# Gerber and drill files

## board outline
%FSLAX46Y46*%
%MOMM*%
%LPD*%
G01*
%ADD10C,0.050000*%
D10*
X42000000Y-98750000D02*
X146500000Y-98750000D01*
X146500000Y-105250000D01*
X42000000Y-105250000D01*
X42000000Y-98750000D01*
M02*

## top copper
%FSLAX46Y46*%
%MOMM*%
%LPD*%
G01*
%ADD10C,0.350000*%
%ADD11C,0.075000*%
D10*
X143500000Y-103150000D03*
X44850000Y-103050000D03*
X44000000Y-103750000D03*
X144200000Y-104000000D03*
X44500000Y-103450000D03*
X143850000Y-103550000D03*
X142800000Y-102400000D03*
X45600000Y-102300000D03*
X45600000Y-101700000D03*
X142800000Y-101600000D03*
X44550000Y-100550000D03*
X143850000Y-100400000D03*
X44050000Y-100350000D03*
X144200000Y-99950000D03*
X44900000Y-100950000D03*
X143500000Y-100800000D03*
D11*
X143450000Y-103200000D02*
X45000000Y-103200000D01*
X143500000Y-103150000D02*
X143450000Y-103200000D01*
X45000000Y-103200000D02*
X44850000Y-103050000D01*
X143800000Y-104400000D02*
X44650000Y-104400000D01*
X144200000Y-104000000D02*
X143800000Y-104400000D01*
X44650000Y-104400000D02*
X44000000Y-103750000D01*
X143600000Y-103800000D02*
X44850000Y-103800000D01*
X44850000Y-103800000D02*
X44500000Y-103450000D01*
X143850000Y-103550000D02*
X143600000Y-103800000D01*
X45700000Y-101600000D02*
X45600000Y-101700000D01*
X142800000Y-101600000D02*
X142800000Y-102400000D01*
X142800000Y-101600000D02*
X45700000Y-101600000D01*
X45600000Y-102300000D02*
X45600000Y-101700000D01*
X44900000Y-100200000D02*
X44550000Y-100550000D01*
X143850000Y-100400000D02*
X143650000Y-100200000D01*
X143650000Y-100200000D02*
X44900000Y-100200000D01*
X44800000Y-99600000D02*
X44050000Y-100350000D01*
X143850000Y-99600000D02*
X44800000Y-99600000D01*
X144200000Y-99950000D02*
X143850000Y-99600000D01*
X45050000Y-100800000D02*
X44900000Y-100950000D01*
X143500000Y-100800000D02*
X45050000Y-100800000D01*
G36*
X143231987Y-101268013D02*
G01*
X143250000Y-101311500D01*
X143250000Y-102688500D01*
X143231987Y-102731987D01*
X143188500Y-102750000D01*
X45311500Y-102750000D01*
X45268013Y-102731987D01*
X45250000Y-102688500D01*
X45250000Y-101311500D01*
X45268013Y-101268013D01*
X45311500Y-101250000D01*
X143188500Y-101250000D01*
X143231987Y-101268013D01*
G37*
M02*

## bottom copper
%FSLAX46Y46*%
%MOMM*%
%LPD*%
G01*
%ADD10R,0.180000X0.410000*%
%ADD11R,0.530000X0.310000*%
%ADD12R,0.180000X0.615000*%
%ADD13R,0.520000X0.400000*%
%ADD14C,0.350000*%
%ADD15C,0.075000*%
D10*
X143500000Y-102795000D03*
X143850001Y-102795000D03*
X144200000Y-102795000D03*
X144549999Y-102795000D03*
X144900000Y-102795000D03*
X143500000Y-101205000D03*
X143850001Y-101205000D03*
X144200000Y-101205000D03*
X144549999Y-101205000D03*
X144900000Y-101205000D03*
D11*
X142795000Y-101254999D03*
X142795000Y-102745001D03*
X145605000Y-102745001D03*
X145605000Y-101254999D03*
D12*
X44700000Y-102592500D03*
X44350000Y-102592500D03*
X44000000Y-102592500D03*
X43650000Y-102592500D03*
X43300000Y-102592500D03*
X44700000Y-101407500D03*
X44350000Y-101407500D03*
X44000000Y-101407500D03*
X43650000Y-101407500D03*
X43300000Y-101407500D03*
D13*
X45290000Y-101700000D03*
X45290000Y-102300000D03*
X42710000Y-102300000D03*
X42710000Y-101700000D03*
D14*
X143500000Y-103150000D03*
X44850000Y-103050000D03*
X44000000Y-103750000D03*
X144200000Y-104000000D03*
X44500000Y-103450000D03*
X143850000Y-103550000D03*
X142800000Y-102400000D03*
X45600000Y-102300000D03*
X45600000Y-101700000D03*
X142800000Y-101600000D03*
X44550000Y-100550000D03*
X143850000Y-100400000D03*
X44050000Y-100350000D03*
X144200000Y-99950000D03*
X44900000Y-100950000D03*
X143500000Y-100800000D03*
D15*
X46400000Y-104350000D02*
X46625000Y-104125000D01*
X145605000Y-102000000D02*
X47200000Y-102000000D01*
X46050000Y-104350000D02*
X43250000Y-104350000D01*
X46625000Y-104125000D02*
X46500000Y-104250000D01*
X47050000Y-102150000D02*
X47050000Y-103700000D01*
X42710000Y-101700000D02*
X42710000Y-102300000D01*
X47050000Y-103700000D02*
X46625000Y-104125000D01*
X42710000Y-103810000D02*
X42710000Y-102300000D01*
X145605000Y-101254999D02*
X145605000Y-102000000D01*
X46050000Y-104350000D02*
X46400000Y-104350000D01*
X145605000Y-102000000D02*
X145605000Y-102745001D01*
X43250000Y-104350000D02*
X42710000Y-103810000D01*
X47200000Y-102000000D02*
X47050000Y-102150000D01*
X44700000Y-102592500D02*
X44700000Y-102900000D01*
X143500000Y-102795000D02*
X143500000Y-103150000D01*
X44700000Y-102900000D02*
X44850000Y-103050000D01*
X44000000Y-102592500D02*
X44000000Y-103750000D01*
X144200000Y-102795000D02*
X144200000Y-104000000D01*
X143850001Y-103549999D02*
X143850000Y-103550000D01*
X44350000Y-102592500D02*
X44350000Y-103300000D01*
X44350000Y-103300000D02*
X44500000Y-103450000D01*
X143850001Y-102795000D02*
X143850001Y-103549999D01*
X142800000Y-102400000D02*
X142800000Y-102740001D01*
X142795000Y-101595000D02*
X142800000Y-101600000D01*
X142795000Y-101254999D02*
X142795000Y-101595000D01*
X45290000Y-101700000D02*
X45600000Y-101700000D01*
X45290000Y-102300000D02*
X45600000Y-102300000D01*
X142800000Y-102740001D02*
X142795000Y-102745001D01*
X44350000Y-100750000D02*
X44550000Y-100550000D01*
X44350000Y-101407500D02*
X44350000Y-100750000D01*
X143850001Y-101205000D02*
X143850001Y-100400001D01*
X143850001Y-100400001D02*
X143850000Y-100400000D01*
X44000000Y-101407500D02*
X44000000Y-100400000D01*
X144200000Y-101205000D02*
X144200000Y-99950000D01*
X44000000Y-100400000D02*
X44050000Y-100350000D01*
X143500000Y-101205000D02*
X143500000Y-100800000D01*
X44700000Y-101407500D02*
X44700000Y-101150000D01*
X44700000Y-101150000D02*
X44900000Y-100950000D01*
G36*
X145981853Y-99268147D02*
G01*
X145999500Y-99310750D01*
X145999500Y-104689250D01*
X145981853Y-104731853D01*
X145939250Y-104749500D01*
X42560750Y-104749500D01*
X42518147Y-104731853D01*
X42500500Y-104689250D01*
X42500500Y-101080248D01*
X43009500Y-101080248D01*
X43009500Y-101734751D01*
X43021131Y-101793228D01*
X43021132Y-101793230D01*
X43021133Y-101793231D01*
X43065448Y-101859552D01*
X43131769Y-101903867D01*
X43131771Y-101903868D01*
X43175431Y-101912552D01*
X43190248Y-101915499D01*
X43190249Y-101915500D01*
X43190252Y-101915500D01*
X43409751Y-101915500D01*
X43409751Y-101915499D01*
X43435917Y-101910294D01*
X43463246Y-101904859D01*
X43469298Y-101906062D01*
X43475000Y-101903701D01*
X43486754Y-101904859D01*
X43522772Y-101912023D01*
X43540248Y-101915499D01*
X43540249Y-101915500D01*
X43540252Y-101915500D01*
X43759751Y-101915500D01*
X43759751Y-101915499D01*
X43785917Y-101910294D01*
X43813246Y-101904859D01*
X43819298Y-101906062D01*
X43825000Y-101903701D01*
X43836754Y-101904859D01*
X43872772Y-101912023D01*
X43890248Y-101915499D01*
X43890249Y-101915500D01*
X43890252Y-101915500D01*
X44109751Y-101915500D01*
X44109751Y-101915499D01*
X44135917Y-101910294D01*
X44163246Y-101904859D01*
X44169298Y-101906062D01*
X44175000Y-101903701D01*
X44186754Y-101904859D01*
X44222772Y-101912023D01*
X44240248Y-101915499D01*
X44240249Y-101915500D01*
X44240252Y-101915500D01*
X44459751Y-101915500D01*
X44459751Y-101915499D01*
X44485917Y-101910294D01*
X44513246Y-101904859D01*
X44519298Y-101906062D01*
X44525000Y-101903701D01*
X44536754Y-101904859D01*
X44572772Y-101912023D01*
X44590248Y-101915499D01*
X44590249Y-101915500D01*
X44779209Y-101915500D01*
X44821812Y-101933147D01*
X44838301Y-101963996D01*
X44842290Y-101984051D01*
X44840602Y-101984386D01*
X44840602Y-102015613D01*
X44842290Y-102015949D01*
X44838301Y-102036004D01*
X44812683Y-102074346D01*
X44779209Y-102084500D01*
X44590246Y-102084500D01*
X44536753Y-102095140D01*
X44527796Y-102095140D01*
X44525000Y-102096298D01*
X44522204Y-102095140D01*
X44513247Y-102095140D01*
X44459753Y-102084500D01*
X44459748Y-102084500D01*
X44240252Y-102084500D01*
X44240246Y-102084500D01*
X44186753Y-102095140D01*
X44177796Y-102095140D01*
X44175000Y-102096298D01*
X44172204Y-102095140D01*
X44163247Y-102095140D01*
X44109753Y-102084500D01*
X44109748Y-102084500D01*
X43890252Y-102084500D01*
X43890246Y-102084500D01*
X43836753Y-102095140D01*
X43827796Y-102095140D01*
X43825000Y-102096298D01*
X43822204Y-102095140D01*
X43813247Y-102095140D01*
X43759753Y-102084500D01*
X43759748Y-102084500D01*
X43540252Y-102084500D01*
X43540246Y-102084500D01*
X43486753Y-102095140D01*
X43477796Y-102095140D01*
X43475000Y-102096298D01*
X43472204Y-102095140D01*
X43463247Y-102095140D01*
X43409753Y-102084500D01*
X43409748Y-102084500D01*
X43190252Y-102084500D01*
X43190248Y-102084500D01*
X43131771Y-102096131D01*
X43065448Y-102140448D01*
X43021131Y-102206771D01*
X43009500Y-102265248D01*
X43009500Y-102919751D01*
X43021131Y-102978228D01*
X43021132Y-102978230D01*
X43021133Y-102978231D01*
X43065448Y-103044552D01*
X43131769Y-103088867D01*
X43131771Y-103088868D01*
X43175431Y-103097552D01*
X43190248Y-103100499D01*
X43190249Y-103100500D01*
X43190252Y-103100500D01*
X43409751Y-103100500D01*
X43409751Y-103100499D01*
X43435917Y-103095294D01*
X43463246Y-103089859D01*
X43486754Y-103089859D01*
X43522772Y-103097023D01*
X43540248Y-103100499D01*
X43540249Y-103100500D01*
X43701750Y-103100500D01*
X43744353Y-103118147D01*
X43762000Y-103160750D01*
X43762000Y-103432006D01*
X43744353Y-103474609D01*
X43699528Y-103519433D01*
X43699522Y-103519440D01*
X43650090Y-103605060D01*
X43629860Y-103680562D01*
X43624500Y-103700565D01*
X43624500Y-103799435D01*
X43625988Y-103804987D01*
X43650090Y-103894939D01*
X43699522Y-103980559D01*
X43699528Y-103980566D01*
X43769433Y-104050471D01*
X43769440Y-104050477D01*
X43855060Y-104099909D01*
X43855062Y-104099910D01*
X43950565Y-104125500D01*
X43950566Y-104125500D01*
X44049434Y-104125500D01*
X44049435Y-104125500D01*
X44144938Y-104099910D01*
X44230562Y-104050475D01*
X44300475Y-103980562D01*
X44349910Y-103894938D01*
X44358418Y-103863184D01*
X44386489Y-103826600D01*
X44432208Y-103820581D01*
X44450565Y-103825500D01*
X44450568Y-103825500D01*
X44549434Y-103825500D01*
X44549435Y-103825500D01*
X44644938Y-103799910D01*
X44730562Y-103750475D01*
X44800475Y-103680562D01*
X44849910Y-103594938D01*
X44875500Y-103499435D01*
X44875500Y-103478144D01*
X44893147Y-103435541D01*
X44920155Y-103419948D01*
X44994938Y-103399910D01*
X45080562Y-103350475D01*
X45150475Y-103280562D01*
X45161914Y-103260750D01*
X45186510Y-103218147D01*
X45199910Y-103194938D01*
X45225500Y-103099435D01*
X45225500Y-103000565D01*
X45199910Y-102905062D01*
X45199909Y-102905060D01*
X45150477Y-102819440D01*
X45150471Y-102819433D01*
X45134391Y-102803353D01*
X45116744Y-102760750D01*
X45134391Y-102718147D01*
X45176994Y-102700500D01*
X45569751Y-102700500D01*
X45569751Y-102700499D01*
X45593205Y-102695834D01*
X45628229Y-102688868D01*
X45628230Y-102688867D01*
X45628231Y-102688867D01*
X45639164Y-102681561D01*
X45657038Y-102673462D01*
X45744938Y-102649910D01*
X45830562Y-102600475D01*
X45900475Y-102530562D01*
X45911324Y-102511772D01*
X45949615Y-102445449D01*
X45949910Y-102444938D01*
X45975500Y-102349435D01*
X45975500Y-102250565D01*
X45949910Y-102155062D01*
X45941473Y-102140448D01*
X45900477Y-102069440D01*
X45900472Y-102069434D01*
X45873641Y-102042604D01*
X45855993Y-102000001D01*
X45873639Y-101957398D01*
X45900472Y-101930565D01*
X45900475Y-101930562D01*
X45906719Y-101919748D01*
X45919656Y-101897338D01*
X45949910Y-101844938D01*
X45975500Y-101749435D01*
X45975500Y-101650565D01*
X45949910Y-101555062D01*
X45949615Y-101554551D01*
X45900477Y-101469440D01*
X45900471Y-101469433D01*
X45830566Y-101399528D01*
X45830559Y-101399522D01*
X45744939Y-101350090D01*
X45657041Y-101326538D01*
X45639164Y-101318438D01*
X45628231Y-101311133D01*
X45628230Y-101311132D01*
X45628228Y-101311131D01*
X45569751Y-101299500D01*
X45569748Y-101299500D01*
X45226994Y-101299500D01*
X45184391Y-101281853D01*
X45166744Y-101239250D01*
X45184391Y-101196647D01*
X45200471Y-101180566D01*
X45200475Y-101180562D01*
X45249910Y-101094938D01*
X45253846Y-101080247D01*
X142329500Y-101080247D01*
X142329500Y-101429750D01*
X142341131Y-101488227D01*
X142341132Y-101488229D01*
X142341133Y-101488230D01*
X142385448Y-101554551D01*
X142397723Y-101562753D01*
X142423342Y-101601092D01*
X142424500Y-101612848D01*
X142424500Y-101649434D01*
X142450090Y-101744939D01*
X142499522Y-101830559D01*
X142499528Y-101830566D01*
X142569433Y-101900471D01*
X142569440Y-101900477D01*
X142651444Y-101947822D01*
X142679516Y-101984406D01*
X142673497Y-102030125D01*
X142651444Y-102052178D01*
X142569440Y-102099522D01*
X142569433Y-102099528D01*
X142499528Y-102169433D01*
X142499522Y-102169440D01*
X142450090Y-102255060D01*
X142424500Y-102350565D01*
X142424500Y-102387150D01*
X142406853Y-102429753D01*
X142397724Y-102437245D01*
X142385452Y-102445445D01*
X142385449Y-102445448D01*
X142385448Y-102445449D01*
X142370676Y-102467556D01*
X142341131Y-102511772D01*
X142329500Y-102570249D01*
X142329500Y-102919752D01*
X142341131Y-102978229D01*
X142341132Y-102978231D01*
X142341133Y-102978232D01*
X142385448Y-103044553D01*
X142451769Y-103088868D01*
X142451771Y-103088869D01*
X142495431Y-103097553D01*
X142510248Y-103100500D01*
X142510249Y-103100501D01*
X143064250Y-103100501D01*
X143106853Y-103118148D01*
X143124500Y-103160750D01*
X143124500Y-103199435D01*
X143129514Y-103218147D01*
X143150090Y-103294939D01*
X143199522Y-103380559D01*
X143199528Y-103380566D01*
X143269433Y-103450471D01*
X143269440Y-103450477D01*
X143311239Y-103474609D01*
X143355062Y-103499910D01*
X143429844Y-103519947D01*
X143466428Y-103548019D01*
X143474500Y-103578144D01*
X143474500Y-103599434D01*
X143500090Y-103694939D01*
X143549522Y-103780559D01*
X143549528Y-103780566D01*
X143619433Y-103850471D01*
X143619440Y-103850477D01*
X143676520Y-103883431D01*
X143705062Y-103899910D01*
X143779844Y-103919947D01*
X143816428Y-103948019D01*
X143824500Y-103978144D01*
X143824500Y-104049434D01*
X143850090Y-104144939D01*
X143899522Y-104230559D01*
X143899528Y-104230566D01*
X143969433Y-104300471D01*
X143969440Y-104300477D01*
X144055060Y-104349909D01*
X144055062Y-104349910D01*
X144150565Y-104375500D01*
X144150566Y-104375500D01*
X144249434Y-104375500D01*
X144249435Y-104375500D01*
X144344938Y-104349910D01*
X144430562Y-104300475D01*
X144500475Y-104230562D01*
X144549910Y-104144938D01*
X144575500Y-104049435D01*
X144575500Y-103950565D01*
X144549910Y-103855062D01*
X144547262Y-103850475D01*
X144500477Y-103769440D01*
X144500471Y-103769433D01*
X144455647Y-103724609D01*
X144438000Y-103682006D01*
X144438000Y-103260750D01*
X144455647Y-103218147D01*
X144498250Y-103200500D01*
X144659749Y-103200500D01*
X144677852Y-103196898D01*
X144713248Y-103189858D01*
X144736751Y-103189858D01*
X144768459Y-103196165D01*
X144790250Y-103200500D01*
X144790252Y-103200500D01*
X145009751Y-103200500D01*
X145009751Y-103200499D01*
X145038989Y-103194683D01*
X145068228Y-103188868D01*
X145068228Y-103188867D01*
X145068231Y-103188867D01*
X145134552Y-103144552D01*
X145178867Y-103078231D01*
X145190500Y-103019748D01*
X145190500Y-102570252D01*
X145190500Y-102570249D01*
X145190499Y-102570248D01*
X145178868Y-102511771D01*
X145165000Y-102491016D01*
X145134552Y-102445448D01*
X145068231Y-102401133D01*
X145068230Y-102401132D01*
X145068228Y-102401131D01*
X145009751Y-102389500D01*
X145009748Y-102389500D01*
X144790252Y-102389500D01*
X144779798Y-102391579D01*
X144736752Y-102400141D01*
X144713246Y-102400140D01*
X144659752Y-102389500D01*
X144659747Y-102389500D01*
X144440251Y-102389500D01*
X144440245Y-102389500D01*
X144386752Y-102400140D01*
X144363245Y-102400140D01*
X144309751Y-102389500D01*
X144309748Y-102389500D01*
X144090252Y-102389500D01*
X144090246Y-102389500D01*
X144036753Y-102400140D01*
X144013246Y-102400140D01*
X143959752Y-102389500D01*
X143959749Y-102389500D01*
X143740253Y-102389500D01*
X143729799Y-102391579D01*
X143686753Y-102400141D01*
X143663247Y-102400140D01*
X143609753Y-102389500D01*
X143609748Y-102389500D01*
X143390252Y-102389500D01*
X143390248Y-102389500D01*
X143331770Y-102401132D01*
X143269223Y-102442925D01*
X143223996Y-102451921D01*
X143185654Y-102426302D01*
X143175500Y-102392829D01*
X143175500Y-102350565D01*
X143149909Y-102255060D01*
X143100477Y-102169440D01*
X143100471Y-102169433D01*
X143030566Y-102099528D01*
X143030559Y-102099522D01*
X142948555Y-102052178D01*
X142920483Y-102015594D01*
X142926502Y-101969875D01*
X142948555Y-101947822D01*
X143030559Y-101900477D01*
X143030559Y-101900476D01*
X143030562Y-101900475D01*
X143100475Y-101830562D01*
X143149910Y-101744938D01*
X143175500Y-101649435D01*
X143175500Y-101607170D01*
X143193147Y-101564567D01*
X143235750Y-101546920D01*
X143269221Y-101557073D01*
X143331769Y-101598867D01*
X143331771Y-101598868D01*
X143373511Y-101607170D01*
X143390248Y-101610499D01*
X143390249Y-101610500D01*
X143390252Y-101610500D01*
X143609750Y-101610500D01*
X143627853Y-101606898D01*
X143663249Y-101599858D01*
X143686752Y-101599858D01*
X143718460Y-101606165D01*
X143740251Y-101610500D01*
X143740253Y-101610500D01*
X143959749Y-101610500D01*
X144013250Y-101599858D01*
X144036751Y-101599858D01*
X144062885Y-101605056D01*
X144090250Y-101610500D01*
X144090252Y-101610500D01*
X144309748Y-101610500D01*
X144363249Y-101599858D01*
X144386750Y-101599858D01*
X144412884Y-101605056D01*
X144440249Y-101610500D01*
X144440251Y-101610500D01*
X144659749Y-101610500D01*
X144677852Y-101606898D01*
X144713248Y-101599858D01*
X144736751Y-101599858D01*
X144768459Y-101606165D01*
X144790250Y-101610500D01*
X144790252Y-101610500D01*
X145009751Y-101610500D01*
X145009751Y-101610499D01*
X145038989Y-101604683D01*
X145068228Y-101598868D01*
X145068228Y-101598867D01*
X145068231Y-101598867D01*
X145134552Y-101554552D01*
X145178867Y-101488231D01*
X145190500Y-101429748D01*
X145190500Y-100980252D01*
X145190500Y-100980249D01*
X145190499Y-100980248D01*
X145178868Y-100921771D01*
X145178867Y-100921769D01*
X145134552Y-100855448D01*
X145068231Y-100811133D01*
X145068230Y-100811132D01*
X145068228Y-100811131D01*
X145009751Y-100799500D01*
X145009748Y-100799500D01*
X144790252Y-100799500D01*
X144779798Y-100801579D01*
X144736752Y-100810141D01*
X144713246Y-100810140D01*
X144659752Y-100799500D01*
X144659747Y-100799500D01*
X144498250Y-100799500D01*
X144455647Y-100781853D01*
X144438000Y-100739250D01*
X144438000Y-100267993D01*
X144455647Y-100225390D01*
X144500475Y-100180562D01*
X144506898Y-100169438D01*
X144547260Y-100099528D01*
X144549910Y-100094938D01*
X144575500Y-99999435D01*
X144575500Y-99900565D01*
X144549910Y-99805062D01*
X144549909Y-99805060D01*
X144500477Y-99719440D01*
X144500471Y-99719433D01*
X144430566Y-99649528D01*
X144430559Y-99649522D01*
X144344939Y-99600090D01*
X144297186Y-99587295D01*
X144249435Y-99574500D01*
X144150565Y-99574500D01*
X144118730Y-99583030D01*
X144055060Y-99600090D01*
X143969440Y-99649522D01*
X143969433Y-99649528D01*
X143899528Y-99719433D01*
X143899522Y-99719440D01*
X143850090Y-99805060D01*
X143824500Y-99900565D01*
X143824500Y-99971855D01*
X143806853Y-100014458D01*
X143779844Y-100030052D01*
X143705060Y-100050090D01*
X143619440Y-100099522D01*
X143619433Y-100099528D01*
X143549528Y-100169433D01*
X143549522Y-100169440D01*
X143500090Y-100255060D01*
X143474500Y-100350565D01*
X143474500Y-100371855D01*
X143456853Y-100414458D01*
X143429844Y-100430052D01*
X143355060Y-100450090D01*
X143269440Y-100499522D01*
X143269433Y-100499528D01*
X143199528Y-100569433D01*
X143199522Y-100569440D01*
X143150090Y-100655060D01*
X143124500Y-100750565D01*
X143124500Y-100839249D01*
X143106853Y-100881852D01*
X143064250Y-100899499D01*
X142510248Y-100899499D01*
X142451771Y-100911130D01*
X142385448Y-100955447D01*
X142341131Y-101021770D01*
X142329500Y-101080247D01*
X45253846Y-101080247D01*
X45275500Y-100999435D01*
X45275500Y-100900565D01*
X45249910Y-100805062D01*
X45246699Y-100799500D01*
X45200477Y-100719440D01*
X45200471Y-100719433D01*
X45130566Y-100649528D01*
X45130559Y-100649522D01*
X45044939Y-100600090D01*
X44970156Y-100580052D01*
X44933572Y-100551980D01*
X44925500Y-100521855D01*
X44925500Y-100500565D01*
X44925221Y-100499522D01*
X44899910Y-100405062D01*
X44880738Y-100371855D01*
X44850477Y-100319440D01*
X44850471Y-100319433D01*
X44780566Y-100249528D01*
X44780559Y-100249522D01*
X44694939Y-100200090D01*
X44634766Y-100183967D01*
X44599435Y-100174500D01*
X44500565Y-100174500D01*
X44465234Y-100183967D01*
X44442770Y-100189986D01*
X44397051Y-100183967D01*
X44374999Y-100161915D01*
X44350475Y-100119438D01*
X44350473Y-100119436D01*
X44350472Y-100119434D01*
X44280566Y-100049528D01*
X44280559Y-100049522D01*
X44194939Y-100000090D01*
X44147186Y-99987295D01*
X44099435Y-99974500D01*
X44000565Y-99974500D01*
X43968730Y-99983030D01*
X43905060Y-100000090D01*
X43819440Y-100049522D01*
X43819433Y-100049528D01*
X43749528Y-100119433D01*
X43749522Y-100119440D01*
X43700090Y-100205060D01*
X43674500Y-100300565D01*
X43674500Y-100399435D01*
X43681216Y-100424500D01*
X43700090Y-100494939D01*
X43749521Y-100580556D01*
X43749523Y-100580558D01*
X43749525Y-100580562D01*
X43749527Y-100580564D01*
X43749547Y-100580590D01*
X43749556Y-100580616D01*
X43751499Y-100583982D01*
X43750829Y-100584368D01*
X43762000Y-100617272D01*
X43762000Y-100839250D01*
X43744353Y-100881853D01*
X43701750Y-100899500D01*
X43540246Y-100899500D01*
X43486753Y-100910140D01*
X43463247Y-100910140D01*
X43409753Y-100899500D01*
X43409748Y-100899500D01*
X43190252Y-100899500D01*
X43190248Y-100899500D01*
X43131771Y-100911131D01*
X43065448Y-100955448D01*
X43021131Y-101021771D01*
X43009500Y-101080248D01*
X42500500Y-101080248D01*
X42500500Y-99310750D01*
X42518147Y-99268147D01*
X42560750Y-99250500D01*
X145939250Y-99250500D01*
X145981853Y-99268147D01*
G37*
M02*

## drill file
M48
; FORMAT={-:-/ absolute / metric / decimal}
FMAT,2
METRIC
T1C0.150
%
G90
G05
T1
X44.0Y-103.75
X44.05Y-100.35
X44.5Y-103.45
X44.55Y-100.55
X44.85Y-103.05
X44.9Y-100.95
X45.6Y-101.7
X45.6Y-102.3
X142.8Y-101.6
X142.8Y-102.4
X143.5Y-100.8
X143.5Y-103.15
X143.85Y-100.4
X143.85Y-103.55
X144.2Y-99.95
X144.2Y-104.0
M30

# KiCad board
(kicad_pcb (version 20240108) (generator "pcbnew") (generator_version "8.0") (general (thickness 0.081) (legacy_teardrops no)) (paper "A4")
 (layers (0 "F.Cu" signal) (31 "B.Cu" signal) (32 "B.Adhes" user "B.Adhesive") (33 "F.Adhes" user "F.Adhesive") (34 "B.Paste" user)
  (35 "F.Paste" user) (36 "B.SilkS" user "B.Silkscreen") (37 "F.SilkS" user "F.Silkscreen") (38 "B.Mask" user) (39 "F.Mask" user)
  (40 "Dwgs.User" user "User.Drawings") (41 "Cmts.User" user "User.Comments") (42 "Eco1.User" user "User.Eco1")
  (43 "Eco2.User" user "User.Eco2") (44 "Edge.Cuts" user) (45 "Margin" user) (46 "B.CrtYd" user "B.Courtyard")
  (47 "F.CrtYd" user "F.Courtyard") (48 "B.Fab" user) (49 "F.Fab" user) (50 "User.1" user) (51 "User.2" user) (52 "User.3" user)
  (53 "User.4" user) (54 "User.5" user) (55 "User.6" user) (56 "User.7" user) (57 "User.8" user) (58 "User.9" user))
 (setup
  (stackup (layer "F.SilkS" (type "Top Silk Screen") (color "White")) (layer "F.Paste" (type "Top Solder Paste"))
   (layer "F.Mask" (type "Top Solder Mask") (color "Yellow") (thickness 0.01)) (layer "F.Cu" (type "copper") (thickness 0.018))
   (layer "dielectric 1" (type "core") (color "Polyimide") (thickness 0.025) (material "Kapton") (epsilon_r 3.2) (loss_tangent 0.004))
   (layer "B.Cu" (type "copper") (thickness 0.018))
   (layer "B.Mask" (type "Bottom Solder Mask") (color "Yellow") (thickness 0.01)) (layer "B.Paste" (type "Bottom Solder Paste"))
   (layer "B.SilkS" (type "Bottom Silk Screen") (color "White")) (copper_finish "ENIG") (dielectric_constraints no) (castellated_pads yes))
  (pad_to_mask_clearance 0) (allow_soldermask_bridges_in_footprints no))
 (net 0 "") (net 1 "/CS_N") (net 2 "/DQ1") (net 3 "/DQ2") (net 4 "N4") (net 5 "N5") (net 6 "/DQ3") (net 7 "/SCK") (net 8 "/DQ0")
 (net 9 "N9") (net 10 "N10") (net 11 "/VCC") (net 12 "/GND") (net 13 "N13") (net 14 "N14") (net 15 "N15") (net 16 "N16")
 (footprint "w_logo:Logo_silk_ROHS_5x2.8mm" (layer "F.Cu") (at 106.5 102.25)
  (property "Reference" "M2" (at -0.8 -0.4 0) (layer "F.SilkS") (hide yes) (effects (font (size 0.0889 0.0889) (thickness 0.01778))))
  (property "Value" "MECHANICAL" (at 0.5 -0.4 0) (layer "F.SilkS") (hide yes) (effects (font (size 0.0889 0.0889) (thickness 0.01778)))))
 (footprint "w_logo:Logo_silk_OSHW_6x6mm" (layer "F.Cu") (at 74.005 101.444565)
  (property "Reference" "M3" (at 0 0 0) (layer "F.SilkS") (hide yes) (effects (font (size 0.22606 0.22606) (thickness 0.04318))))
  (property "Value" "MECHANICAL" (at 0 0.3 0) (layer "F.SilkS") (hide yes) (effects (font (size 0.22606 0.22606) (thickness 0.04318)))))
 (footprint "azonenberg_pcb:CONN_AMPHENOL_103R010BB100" (layer "B.Cu") (at 144.2 102)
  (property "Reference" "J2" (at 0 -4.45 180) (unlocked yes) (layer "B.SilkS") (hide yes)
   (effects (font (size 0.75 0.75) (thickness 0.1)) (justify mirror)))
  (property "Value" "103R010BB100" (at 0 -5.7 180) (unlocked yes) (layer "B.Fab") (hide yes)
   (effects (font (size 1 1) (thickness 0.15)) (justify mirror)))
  (pad "1" smd rect (at -0.7 0.795) (size 0.18 0.41) (layers "B.Cu" "B.Paste" "B.Mask") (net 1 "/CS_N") (thermal_bridge_angle 45))
  (pad "2" smd rect (at -0.349999 0.795) (size 0.18 0.41) (layers "B.Cu" "B.Paste" "B.Mask") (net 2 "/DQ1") (thermal_bridge_angle 45))
  (pad "3" smd rect (at 0 0.795) (size 0.18 0.41) (layers "B.Cu" "B.Paste" "B.Mask") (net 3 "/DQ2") (thermal_bridge_angle 45))
  (pad "4" smd rect (at 0.349999 0.795) (size 0.18 0.41) (layers "B.Cu" "B.Paste" "B.Mask") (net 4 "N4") (thermal_bridge_angle 45))
  (pad "5" smd rect (at 0.7 0.795) (size 0.18 0.41) (layers "B.Cu" "B.Paste" "B.Mask") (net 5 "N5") (thermal_bridge_angle 45))
  (pad "6" smd rect (at -0.7 -0.795) (size 0.18 0.41) (layers "B.Cu" "B.Paste" "B.Mask") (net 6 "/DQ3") (thermal_bridge_angle 45))
  (pad "7" smd rect (at -0.349999 -0.795) (size 0.18 0.41) (layers "B.Cu" "B.Paste" "B.Mask") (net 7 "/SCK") (thermal_bridge_angle 45))
  (pad "8" smd rect (at 0 -0.795) (size 0.18 0.41) (layers "B.Cu" "B.Paste" "B.Mask") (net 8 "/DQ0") (thermal_bridge_angle 45))
  (pad "9" smd rect (at 0.349999 -0.795) (size 0.18 0.41) (layers "B.Cu" "B.Paste" "B.Mask") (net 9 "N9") (thermal_bridge_angle 45))
  (pad "10" smd rect (at 0.7 -0.795) (size 0.18 0.41) (layers "B.Cu" "B.Paste" "B.Mask") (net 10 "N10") (thermal_bridge_angle 45))
  (pad "11" smd rect (at -1.405 -0.745001) (size 0.53 0.31) (layers "B.Cu" "B.Paste" "B.Mask") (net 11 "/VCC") (thermal_bridge_angle 45))
  (pad "12" smd rect (at -1.405 0.745001) (size 0.53 0.31) (layers "B.Cu" "B.Paste" "B.Mask") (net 11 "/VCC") (thermal_bridge_angle 45))
  (pad "13" smd rect (at 1.405 0.745001) (size 0.53 0.31) (layers "B.Cu" "B.Paste" "B.Mask") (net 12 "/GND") (thermal_bridge_angle 45))
  (pad "14" smd rect (at 1.405 -0.745001) (size 0.53 0.31) (layers "B.Cu" "B.Paste" "B.Mask") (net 12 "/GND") (thermal_bridge_angle 45)))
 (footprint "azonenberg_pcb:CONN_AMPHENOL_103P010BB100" (layer "B.Cu") (at 44 102 180)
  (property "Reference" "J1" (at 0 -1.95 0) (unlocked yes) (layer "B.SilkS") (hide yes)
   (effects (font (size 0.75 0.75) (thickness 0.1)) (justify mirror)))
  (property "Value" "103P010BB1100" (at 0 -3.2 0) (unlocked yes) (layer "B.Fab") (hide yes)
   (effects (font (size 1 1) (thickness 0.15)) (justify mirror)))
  (pad "1" smd rect (at -0.7 -0.5925 180) (size 0.18 0.615) (layers "B.Cu" "B.Paste" "B.Mask") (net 1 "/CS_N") (thermal_bridge_angle 45))
  (pad "2" smd rect (at -0.35 -0.5925 180) (size 0.18 0.615) (layers "B.Cu" "B.Paste" "B.Mask") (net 2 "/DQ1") (thermal_bridge_angle 45))
  (pad "3" smd rect (at 0 -0.5925 180) (size 0.18 0.615) (layers "B.Cu" "B.Paste" "B.Mask") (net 3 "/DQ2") (thermal_bridge_angle 45))
  (pad "4" smd rect (at 0.35 -0.5925 180) (size 0.18 0.615) (layers "B.Cu" "B.Paste" "B.Mask") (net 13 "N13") (thermal_bridge_angle 45))
  (pad "5" smd rect (at 0.7 -0.5925 180) (size 0.18 0.615) (layers "B.Cu" "B.Paste" "B.Mask") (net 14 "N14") (thermal_bridge_angle 45))
  (pad "6" smd rect (at -0.7 0.5925 180) (size 0.18 0.615) (layers "B.Cu" "B.Paste" "B.Mask") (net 6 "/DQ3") (thermal_bridge_angle 45))
  (pad "7" smd rect (at -0.35 0.5925 180) (size 0.18 0.615) (layers "B.Cu" "B.Paste" "B.Mask") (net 7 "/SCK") (thermal_bridge_angle 45))
  (pad "8" smd rect (at 0 0.5925 180) (size 0.18 0.615) (layers "B.Cu" "B.Paste" "B.Mask") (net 8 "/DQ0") (thermal_bridge_angle 45))
  (pad "9" smd rect (at 0.35 0.5925 180) (size 0.18 0.615) (layers "B.Cu" "B.Paste" "B.Mask") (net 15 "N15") (thermal_bridge_angle 45))
  (pad "10" smd rect (at 0.7 0.5925 180) (size 0.18 0.615) (layers "B.Cu" "B.Paste" "B.Mask") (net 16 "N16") (thermal_bridge_angle 45))
  (pad "11" smd rect (at -1.29 0.3 180) (size 0.52 0.4) (layers "B.Cu" "B.Paste" "B.Mask") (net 11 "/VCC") (thermal_bridge_angle 45))
  (pad "12" smd rect (at -1.29 -0.3 180) (size 0.52 0.4) (layers "B.Cu" "B.Paste" "B.Mask") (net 11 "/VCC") (thermal_bridge_angle 45))
  (pad "13" smd rect (at 1.29 -0.3 180) (size 0.52 0.4) (layers "B.Cu" "B.Paste" "B.Mask") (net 12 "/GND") (thermal_bridge_angle 45))
  (pad "14" smd rect (at 1.29 0.3 180) (size 0.52 0.4) (layers "B.Cu" "B.Paste" "B.Mask") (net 12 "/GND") (thermal_bridge_angle 45)))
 (gr_rect (start 42 98.75) (end 146.5 105.25) (stroke (width 0.05) (type default)) (fill none) (layer "Edge.Cuts"))
 (segment (start 46.4 104.35) (end 46.625 104.125) (width 0.075) (layer "B.Cu") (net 12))
 (segment (start 145.605 102) (end 47.2 102) (width 0.075) (layer "B.Cu") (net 12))
 (segment (start 46.05 104.35) (end 43.25 104.35) (width 0.075) (layer "B.Cu") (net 12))
 (segment (start 46.625 104.125) (end 46.5 104.25) (width 0.075) (layer "B.Cu") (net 12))
 (segment (start 47.05 102.15) (end 47.05 103.7) (width 0.075) (layer "B.Cu") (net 12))
 (segment (start 42.71 101.7) (end 42.71 102.3) (width 0.075) (layer "B.Cu") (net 12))
 (segment (start 47.05 103.7) (end 46.625 104.125) (width 0.075) (layer "B.Cu") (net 12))
 (segment (start 42.71 103.81) (end 42.71 102.3) (width 0.075) (layer "B.Cu") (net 12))
 (segment (start 145.605 101.254999) (end 145.605 102) (width 0.075) (layer "B.Cu") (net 12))
 (segment (start 46.05 104.35) (end 46.4 104.35) (width 0.075) (layer "B.Cu") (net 12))
 (segment (start 145.605 102) (end 145.605 102.745001) (width 0.075) (layer "B.Cu") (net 12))
 (segment (start 43.25 104.35) (end 42.71 103.81) (width 0.075) (layer "B.Cu") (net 12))
 (segment (start 47.2 102) (end 47.05 102.15) (width 0.075) (layer "B.Cu") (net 12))
 (segment (start 143.45 103.2) (end 45 103.2) (width 0.075) (layer "F.Cu") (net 1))
 (segment (start 143.5 103.15) (end 143.45 103.2) (width 0.075) (layer "F.Cu") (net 1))
 (segment (start 45 103.2) (end 44.85 103.05) (width 0.075) (layer "F.Cu") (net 1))
 (via (at 143.5 103.15) (size 0.35) (drill 0.15) (layers "F.Cu" "B.Cu") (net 1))
 (via (at 44.85 103.05) (size 0.35) (drill 0.15) (layers "F.Cu" "B.Cu") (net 1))
 (segment (start 44.7 102.5925) (end 44.7 102.9) (width 0.075) (layer "B.Cu") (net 1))
 (segment (start 143.5 102.795) (end 143.5 103.15) (width 0.075) (layer "B.Cu") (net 1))
 (segment (start 44.7 102.9) (end 44.85 103.05) (width 0.075) (layer "B.Cu") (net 1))
 (segment (start 143.8 104.4) (end 44.65 104.4) (width 0.075) (layer "F.Cu") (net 3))
 (segment (start 144.2 104) (end 143.8 104.4) (width 0.075) (layer "F.Cu") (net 3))
 (segment (start 44.65 104.4) (end 44 103.75) (width 0.075) (layer "F.Cu") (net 3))
 (via (at 44 103.75) (size 0.35) (drill 0.15) (layers "F.Cu" "B.Cu") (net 3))
 (via (at 144.2 104) (size 0.35) (drill 0.15) (layers "F.Cu" "B.Cu") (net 3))
 (segment (start 44 102.5925) (end 44 103.75) (width 0.075) (layer "B.Cu") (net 3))
 (segment (start 144.2 102.795) (end 144.2 104) (width 0.075) (layer "B.Cu") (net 3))
 (segment (start 143.6 103.8) (end 44.85 103.8) (width 0.075) (layer "F.Cu") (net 2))
 (segment (start 44.85 103.8) (end 44.5 103.45) (width 0.075) (layer "F.Cu") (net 2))
 (segment (start 143.85 103.55) (end 143.6 103.8) (width 0.075) (layer "F.Cu") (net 2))
 (via (at 44.5 103.45) (size 0.35) (drill 0.15) (layers "F.Cu" "B.Cu") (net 2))
 (via (at 143.85 103.55) (size 0.35) (drill 0.15) (layers "F.Cu" "B.Cu") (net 2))
 (segment (start 143.850001 103.549999) (end 143.85 103.55) (width 0.075) (layer "B.Cu") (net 2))
 (segment (start 44.35 102.5925) (end 44.35 103.3) (width 0.075) (layer "B.Cu") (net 2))
 (segment (start 44.35 103.3) (end 44.5 103.45) (width 0.075) (layer "B.Cu") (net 2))
 (segment (start 143.850001 102.795) (end 143.850001 103.549999) (width 0.075) (layer "B.Cu") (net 2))
 (segment (start 45.7 101.6) (end 45.6 101.7) (width 0.075) (layer "F.Cu") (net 11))
 (segment (start 142.8 101.6) (end 142.8 102.4) (width 0.075) (layer "F.Cu") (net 11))
 (segment (start 142.8 101.6) (end 45.7 101.6) (width 0.075) (layer "F.Cu") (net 11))
 (segment (start 45.6 102.3) (end 45.6 101.7) (width 0.075) (layer "F.Cu") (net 11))
 (via (at 142.8 102.4) (size 0.35) (drill 0.15) (layers "F.Cu" "B.Cu") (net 11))
 (via (at 45.6 102.3) (size 0.35) (drill 0.15) (layers "F.Cu" "B.Cu") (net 11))
 (via (at 45.6 101.7) (size 0.35) (drill 0.15) (layers "F.Cu" "B.Cu") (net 11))
 (via (at 142.8 101.6) (size 0.35) (drill 0.15) (layers "F.Cu" "B.Cu") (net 11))
 (segment (start 142.8 102.4) (end 142.8 102.740001) (width 0.075) (layer "B.Cu") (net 11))
 (segment (start 142.795 101.595) (end 142.8 101.6) (width 0.075) (layer "B.Cu") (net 11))
 (segment (start 142.795 101.254999) (end 142.795 101.595) (width 0.075) (layer "B.Cu") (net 11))
 (segment (start 45.29 101.7) (end 45.6 101.7) (width 0.075) (layer "B.Cu") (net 11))
 (segment (start 45.29 102.3) (end 45.6 102.3) (width 0.075) (layer "B.Cu") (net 11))
 (segment (start 142.8 102.740001) (end 142.795 102.745001) (width 0.075) (layer "B.Cu") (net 11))
 (segment (start 44.9 100.2) (end 44.55 100.55) (width 0.075) (layer "F.Cu") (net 7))
 (segment (start 143.85 100.4) (end 143.65 100.2) (width 0.075) (layer "F.Cu") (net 7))
 (segment (start 143.65 100.2) (end 44.9 100.2) (width 0.075) (layer "F.Cu") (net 7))
 (via (at 44.55 100.55) (size 0.35) (drill 0.15) (layers "F.Cu" "B.Cu") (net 7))
 (via (at 143.85 100.4) (size 0.35) (drill 0.15) (layers "F.Cu" "B.Cu") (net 7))
 (segment (start 44.35 100.75) (end 44.55 100.55) (width 0.075) (layer "B.Cu") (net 7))
 (segment (start 44.35 101.4075) (end 44.35 100.75) (width 0.075) (layer "B.Cu") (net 7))
 (segment (start 143.850001 101.205) (end 143.850001 100.400001) (width 0.075) (layer "B.Cu") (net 7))
 (segment (start 143.850001 100.400001) (end 143.85 100.4) (width 0.075) (layer "B.Cu") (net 7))
 (segment (start 44.8 99.6) (end 44.05 100.35) (width 0.075) (layer "F.Cu") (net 8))
 (segment (start 143.85 99.6) (end 44.8 99.6) (width 0.075) (layer "F.Cu") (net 8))
 (segment (start 144.2 99.95) (end 143.85 99.6) (width 0.075) (layer "F.Cu") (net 8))
 (via (at 44.05 100.35) (size 0.35) (drill 0.15) (layers "F.Cu" "B.Cu") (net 8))
 (via (at 144.2 99.95) (size 0.35) (drill 0.15) (layers "F.Cu" "B.Cu") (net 8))
 (segment (start 44 101.4075) (end 44 100.4) (width 0.075) (layer "B.Cu") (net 8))
 (segment (start 144.2 101.205) (end 144.2 99.95) (width 0.075) (layer "B.Cu") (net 8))
 (segment (start 44 100.4) (end 44.05 100.35) (width 0.075) (layer "B.Cu") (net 8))
 (segment (start 45.05 100.8) (end 44.9 100.95) (width 0.075) (layer "F.Cu") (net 6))
 (segment (start 143.5 100.8) (end 45.05 100.8) (width 0.075) (layer "F.Cu") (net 6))
 (via (at 44.9 100.95) (size 0.35) (drill 0.15) (layers "F.Cu" "B.Cu") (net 6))
 (via (at 143.5 100.8) (size 0.35) (drill 0.15) (layers "F.Cu" "B.Cu") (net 6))
 (segment (start 143.5 101.205) (end 143.5 100.8) (width 0.075) (layer "B.Cu") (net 6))
 (segment (start 44.7 101.4075) (end 44.7 101.15) (width 0.075) (layer "B.Cu") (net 6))
 (segment (start 44.7 101.15) (end 44.9 100.95) (width 0.075) (layer "B.Cu") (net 6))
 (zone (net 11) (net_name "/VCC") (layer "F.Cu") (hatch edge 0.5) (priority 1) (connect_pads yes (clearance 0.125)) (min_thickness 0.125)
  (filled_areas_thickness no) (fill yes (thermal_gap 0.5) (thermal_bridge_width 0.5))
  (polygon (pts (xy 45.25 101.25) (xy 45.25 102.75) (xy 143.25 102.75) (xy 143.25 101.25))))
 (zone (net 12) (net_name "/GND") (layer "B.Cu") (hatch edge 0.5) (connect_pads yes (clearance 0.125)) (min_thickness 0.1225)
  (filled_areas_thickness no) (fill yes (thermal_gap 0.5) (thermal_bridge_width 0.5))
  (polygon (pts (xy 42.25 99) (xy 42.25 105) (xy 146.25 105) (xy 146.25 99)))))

